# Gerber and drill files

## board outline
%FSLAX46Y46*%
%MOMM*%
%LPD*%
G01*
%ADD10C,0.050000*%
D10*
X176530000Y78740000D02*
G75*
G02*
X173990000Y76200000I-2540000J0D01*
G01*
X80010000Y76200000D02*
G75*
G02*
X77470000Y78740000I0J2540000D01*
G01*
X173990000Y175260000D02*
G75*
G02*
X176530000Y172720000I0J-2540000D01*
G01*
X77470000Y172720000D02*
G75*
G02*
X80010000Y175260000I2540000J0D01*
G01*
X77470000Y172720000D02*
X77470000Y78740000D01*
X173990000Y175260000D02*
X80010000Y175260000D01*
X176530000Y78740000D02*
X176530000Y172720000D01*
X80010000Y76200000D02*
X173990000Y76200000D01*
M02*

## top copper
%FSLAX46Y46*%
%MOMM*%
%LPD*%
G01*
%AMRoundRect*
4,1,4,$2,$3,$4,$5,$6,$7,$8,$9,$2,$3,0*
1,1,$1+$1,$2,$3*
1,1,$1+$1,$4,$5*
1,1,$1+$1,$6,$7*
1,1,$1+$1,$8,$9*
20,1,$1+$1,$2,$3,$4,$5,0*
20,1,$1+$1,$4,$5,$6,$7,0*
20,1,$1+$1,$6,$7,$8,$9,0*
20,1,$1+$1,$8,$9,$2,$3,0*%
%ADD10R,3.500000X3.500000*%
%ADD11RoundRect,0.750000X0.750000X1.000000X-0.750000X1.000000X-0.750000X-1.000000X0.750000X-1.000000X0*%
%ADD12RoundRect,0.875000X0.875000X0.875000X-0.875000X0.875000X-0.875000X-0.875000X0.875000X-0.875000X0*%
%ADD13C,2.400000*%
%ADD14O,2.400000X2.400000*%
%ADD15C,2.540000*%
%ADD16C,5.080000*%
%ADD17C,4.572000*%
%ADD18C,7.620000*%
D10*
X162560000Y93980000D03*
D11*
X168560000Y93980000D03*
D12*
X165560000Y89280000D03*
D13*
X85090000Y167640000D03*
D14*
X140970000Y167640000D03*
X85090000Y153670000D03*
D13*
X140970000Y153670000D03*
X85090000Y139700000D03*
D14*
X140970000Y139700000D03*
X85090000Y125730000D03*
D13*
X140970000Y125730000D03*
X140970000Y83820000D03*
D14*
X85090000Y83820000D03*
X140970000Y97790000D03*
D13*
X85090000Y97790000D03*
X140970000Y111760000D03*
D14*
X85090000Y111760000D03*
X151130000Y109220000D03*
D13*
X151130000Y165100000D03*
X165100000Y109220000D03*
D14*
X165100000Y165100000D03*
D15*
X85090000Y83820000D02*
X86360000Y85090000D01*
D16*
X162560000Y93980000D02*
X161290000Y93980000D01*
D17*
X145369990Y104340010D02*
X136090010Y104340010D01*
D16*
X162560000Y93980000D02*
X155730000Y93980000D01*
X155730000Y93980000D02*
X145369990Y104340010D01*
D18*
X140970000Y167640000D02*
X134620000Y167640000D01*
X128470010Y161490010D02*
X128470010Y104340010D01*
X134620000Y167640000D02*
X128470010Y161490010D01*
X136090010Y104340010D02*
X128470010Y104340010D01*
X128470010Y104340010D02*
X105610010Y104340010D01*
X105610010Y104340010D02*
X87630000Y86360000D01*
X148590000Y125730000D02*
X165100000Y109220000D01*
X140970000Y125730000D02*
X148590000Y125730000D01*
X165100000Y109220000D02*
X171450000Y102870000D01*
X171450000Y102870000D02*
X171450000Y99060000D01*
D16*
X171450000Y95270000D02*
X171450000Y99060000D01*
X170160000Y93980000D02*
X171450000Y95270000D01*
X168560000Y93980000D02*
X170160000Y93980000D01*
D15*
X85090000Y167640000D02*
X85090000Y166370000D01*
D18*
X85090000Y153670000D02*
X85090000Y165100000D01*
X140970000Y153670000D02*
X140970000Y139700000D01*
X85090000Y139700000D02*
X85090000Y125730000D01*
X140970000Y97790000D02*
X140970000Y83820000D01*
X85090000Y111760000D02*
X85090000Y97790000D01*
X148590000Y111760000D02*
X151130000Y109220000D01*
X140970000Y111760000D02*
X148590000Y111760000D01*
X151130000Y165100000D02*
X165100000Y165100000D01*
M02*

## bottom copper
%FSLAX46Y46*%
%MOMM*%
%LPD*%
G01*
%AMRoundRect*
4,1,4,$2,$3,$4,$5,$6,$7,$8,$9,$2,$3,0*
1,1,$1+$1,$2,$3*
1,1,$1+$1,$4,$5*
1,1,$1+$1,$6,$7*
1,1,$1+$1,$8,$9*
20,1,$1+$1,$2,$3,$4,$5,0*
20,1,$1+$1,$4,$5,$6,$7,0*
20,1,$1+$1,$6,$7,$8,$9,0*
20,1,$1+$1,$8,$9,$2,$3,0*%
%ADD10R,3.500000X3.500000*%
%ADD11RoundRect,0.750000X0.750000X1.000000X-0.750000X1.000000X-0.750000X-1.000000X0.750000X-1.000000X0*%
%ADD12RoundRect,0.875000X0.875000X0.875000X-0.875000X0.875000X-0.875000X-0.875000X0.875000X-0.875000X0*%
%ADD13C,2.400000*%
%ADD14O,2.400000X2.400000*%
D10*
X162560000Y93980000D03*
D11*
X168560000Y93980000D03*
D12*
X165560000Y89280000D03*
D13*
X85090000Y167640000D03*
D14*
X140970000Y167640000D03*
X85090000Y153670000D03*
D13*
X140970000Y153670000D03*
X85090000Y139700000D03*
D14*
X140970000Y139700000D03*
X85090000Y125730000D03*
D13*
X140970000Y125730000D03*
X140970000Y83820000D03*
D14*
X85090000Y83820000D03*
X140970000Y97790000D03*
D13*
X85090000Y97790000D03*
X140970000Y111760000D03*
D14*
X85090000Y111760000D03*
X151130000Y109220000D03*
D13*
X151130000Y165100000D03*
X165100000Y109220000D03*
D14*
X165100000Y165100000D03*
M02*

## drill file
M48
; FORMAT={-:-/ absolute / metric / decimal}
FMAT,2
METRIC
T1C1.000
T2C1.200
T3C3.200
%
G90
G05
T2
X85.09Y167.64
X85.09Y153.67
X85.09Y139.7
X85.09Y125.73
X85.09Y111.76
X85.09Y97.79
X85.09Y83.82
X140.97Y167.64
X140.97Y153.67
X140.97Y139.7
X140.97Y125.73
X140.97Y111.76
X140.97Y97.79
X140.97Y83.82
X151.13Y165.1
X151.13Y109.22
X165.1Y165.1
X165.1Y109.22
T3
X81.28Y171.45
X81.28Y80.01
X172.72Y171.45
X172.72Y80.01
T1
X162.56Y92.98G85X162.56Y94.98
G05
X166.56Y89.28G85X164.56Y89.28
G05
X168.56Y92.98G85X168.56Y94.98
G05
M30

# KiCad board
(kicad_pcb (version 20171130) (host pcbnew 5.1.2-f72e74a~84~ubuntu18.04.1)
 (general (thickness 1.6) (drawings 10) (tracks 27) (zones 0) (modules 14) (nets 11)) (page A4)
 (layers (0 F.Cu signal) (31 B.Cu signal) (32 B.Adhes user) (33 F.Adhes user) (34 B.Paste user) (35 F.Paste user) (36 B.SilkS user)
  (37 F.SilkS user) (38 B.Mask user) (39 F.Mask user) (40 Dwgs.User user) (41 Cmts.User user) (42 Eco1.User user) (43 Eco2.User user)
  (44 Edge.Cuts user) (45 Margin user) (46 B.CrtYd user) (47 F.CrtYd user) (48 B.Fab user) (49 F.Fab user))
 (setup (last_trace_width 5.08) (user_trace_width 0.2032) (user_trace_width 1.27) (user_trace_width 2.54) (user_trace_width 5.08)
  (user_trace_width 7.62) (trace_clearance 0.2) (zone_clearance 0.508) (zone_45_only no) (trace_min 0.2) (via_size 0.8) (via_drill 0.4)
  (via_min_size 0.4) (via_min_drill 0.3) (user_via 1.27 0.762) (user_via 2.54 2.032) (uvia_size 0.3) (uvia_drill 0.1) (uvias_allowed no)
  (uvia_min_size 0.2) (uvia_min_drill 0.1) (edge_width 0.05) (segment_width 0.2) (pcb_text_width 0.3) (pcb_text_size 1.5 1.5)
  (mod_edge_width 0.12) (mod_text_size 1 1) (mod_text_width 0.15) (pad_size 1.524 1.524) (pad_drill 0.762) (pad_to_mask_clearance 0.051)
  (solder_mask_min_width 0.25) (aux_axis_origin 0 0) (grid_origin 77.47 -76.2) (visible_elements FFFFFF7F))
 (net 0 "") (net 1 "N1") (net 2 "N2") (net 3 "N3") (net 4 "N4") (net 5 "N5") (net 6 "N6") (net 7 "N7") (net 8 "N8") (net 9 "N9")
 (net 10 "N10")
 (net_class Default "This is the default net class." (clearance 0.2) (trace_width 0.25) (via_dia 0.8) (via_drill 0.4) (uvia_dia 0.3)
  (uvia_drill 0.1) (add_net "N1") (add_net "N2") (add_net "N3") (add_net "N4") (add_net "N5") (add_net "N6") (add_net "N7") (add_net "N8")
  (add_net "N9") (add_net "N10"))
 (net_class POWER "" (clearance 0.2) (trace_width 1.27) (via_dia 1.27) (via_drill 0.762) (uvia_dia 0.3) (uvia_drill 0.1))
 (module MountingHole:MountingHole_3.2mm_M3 (layer F.Cu) (at 172.72 -80.01)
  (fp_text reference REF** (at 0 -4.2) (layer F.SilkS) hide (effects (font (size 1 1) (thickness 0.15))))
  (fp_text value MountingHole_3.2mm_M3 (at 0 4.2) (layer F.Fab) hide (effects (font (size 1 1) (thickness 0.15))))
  (pad 1 np_thru_hole circle (at 0 0) (size 3.2 3.2) (drill 3.2) (layers *.Cu *.Mask)))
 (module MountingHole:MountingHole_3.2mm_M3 (layer F.Cu) (at 81.28 -80.01)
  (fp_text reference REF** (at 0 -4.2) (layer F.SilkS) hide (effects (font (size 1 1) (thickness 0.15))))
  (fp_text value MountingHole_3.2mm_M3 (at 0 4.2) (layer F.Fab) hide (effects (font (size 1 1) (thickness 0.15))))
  (pad 1 np_thru_hole circle (at 0 0) (size 3.2 3.2) (drill 3.2) (layers *.Cu *.Mask)))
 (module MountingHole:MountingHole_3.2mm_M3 (layer F.Cu) (at 172.72 -171.45)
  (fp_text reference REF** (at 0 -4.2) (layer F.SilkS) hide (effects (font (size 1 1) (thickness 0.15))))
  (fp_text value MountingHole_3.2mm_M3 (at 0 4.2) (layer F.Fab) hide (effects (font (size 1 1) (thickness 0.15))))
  (pad 1 np_thru_hole circle (at 0 0) (size 3.2 3.2) (drill 3.2) (layers *.Cu *.Mask)))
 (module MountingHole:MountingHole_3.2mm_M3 (layer F.Cu) (at 81.28 -171.45)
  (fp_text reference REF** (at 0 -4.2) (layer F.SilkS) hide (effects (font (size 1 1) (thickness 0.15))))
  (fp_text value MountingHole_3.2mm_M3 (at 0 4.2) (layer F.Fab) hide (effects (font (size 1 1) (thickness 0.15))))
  (pad 1 np_thru_hole circle (at 0 0) (size 3.2 3.2) (drill 3.2) (layers *.Cu *.Mask)))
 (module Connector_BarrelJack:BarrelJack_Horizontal (layer B.Cu) (at 162.56 -93.98 180)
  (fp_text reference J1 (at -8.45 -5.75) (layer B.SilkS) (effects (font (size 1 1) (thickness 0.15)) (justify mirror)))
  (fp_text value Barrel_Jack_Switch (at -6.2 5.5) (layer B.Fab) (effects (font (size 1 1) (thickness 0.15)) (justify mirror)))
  (pad 1 thru_hole rect (at 0 0 180) (size 3.5 3.5) (drill oval 1 3) (layers *.Cu *.Mask) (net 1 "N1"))
  (pad 2 thru_hole roundrect (at -6 0 180) (size 3 3.5) (drill oval 1 3) (layers *.Cu *.Mask) (roundrect_rratio 0.25) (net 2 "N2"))
  (pad 3 thru_hole roundrect (at -3 -4.7 180) (size 3.5 3.5) (drill oval 3 1) (layers *.Cu *.Mask) (roundrect_rratio 0.25) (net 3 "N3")))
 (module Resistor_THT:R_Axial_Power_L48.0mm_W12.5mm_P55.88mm (layer F.Cu) (at 85.09 -167.64)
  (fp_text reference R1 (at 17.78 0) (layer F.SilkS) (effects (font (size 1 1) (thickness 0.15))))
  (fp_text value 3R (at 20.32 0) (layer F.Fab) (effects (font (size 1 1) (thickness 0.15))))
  (pad 1 thru_hole circle (at 0 0) (size 2.4 2.4) (drill 1.2) (layers *.Cu *.Mask) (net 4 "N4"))
  (pad 2 thru_hole oval (at 55.88 0) (size 2.4 2.4) (drill 1.2) (layers *.Cu *.Mask) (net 1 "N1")))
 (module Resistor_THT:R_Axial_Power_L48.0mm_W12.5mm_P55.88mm (layer F.Cu) (at 140.97 -153.67 180)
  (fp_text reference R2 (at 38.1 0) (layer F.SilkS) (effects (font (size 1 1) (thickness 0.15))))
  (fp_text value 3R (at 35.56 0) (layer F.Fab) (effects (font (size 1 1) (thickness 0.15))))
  (pad 2 thru_hole oval (at 55.88 0 180) (size 2.4 2.4) (drill 1.2) (layers *.Cu *.Mask) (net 4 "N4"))
  (pad 1 thru_hole circle (at 0 0 180) (size 2.4 2.4) (drill 1.2) (layers *.Cu *.Mask) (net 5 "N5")))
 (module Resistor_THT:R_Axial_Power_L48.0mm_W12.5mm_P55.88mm (layer F.Cu) (at 85.09 -139.7)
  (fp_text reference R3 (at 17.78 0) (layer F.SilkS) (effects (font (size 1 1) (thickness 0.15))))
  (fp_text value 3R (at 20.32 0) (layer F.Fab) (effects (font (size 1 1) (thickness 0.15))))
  (pad 1 thru_hole circle (at 0 0) (size 2.4 2.4) (drill 1.2) (layers *.Cu *.Mask) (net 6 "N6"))
  (pad 2 thru_hole oval (at 55.88 0) (size 2.4 2.4) (drill 1.2) (layers *.Cu *.Mask) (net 5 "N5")))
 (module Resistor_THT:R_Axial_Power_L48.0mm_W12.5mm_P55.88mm (layer F.Cu) (at 140.97 -125.73 180)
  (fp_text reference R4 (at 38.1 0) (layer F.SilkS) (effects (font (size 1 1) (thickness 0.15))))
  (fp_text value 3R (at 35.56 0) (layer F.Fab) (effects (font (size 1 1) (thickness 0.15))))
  (pad 2 thru_hole oval (at 55.88 0 180) (size 2.4 2.4) (drill 1.2) (layers *.Cu *.Mask) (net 6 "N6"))
  (pad 1 thru_hole circle (at 0 0 180) (size 2.4 2.4) (drill 1.2) (layers *.Cu *.Mask) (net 2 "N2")))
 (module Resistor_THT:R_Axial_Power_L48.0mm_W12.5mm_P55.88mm (layer F.Cu) (at 140.97 -83.82 180)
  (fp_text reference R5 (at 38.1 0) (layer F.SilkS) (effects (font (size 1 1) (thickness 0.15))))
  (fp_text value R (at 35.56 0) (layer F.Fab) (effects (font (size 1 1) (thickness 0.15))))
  (pad 1 thru_hole circle (at 0 0 180) (size 2.4 2.4) (drill 1.2) (layers *.Cu *.Mask) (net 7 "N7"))
  (pad 2 thru_hole oval (at 55.88 0 180) (size 2.4 2.4) (drill 1.2) (layers *.Cu *.Mask) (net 1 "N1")))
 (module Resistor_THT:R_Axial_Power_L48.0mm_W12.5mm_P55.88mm (layer F.Cu) (at 85.09 -97.79)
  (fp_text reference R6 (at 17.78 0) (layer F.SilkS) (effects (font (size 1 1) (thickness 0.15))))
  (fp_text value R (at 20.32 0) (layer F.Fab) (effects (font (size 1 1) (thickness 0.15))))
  (pad 2 thru_hole oval (at 55.88 0) (size 2.4 2.4) (drill 1.2) (layers *.Cu *.Mask) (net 7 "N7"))
  (pad 1 thru_hole circle (at 0 0) (size 2.4 2.4) (drill 1.2) (layers *.Cu *.Mask) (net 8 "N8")))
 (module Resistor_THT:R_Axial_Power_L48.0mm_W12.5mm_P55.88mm (layer F.Cu) (at 140.97 -111.76 180)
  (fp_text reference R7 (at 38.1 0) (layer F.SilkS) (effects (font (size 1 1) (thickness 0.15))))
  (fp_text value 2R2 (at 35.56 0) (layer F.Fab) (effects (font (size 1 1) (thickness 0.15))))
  (pad 1 thru_hole circle (at 0 0 180) (size 2.4 2.4) (drill 1.2) (layers *.Cu *.Mask) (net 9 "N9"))
  (pad 2 thru_hole oval (at 55.88 0 180) (size 2.4 2.4) (drill 1.2) (layers *.Cu *.Mask) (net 8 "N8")))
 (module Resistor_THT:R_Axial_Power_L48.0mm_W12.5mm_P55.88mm (layer F.Cu) (at 151.13 -165.1 270)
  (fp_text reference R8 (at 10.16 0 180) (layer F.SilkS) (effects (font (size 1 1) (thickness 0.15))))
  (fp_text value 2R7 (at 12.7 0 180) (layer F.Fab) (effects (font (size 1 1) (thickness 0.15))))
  (pad 2 thru_hole oval (at 55.88 0 270) (size 2.4 2.4) (drill 1.2) (layers *.Cu *.Mask) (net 9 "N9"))
  (pad 1 thru_hole circle (at 0 0 270) (size 2.4 2.4) (drill 1.2) (layers *.Cu *.Mask) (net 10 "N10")))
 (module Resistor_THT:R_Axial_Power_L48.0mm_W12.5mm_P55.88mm (layer F.Cu) (at 165.1 -109.22 90)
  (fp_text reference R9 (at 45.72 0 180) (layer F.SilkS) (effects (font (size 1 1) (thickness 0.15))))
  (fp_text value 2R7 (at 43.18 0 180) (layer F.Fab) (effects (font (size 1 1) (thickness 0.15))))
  (pad 1 thru_hole circle (at 0 0 90) (size 2.4 2.4) (drill 1.2) (layers *.Cu *.Mask) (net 2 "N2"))
  (pad 2 thru_hole oval (at 55.88 0 90) (size 2.4 2.4) (drill 1.2) (layers *.Cu *.Mask) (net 10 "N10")))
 (gr_arc (start 173.99 -78.74) (end 173.99 -76.2) (angle -90) (layer Edge.Cuts) (width 0.05))
 (gr_arc (start 80.01 -78.74) (end 77.47 -78.74) (angle -90) (layer Edge.Cuts) (width 0.05))
 (gr_arc (start 173.99 -172.72) (end 176.53 -172.72) (angle -90) (layer Edge.Cuts) (width 0.05))
 (gr_arc (start 80.01 -172.72) (end 80.01 -175.26) (angle -90) (layer Edge.Cuts) (width 0.05))
 (gr_line (start 77.47 -172.72) (end 77.47 -78.74) (layer Edge.Cuts) (width 0.05))
 (gr_line (start 173.99 -175.26) (end 80.01 -175.26) (layer Edge.Cuts) (width 0.05))
 (gr_line (start 176.53 -78.74) (end 176.53 -172.72) (layer Edge.Cuts) (width 0.05))
 (gr_line (start 80.01 -76.2) (end 173.99 -76.2) (layer Edge.Cuts) (width 0.05))
 (segment (start 85.09 -83.82) (end 86.36 -85.09) (width 2.54) (layer F.Cu) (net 1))
 (segment (start 162.56 -93.98) (end 161.29 -93.98) (width 5.08) (layer F.Cu) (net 1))
 (segment (start 145.36999 -104.34001) (end 136.09001 -104.34001) (width 4.572) (layer F.Cu) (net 1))
 (segment (start 162.56 -93.98) (end 155.73 -93.98) (width 5.08) (layer F.Cu) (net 1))
 (segment (start 155.73 -93.98) (end 145.36999 -104.34001) (width 5.08) (layer F.Cu) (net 1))
 (segment (start 140.97 -167.64) (end 134.62 -167.64) (width 7.62) (layer F.Cu) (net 1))
 (segment (start 128.47001 -161.49001) (end 128.47001 -104.34001) (width 7.62) (layer F.Cu) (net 1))
 (segment (start 134.62 -167.64) (end 128.47001 -161.49001) (width 7.62) (layer F.Cu) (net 1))
 (segment (start 136.09001 -104.34001) (end 128.47001 -104.34001) (width 7.62) (layer F.Cu) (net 1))
 (segment (start 128.47001 -104.34001) (end 105.61001 -104.34001) (width 7.62) (layer F.Cu) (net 1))
 (segment (start 105.61001 -104.34001) (end 87.63 -86.36) (width 7.62) (layer F.Cu) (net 1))
 (segment (start 148.59 -125.73) (end 165.1 -109.22) (width 7.62) (layer F.Cu) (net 2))
 (segment (start 140.97 -125.73) (end 148.59 -125.73) (width 7.62) (layer F.Cu) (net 2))
 (segment (start 165.1 -109.22) (end 171.45 -102.87) (width 7.62) (layer F.Cu) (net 2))
 (segment (start 171.45 -102.87) (end 171.45 -99.06) (width 7.62) (layer F.Cu) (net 2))
 (segment (start 171.45 -95.27) (end 171.45 -99.06) (width 5.08) (layer F.Cu) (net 2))
 (segment (start 170.16 -93.98) (end 171.45 -95.27) (width 5.08) (layer F.Cu) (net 2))
 (segment (start 168.56 -93.98) (end 170.16 -93.98) (width 5.08) (layer F.Cu) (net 2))
 (segment (start 85.09 -167.64) (end 85.09 -166.37) (width 2.54) (layer F.Cu) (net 4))
 (segment (start 85.09 -153.67) (end 85.09 -165.1) (width 7.62) (layer F.Cu) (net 4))
 (segment (start 140.97 -153.67) (end 140.97 -139.7) (width 7.62) (layer F.Cu) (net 5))
 (segment (start 85.09 -139.7) (end 85.09 -125.73) (width 7.62) (layer F.Cu) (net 6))
 (segment (start 140.97 -97.79) (end 140.97 -83.82) (width 7.62) (layer F.Cu) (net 7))
 (segment (start 85.09 -111.76) (end 85.09 -97.79) (width 7.62) (layer F.Cu) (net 8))
 (segment (start 148.59 -111.76) (end 151.13 -109.22) (width 7.62) (layer F.Cu) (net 9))
 (segment (start 140.97 -111.76) (end 148.59 -111.76) (width 7.62) (layer F.Cu) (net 9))
 (segment (start 151.13 -165.1) (end 165.1 -165.1) (width 7.62) (layer F.Cu) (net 10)))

